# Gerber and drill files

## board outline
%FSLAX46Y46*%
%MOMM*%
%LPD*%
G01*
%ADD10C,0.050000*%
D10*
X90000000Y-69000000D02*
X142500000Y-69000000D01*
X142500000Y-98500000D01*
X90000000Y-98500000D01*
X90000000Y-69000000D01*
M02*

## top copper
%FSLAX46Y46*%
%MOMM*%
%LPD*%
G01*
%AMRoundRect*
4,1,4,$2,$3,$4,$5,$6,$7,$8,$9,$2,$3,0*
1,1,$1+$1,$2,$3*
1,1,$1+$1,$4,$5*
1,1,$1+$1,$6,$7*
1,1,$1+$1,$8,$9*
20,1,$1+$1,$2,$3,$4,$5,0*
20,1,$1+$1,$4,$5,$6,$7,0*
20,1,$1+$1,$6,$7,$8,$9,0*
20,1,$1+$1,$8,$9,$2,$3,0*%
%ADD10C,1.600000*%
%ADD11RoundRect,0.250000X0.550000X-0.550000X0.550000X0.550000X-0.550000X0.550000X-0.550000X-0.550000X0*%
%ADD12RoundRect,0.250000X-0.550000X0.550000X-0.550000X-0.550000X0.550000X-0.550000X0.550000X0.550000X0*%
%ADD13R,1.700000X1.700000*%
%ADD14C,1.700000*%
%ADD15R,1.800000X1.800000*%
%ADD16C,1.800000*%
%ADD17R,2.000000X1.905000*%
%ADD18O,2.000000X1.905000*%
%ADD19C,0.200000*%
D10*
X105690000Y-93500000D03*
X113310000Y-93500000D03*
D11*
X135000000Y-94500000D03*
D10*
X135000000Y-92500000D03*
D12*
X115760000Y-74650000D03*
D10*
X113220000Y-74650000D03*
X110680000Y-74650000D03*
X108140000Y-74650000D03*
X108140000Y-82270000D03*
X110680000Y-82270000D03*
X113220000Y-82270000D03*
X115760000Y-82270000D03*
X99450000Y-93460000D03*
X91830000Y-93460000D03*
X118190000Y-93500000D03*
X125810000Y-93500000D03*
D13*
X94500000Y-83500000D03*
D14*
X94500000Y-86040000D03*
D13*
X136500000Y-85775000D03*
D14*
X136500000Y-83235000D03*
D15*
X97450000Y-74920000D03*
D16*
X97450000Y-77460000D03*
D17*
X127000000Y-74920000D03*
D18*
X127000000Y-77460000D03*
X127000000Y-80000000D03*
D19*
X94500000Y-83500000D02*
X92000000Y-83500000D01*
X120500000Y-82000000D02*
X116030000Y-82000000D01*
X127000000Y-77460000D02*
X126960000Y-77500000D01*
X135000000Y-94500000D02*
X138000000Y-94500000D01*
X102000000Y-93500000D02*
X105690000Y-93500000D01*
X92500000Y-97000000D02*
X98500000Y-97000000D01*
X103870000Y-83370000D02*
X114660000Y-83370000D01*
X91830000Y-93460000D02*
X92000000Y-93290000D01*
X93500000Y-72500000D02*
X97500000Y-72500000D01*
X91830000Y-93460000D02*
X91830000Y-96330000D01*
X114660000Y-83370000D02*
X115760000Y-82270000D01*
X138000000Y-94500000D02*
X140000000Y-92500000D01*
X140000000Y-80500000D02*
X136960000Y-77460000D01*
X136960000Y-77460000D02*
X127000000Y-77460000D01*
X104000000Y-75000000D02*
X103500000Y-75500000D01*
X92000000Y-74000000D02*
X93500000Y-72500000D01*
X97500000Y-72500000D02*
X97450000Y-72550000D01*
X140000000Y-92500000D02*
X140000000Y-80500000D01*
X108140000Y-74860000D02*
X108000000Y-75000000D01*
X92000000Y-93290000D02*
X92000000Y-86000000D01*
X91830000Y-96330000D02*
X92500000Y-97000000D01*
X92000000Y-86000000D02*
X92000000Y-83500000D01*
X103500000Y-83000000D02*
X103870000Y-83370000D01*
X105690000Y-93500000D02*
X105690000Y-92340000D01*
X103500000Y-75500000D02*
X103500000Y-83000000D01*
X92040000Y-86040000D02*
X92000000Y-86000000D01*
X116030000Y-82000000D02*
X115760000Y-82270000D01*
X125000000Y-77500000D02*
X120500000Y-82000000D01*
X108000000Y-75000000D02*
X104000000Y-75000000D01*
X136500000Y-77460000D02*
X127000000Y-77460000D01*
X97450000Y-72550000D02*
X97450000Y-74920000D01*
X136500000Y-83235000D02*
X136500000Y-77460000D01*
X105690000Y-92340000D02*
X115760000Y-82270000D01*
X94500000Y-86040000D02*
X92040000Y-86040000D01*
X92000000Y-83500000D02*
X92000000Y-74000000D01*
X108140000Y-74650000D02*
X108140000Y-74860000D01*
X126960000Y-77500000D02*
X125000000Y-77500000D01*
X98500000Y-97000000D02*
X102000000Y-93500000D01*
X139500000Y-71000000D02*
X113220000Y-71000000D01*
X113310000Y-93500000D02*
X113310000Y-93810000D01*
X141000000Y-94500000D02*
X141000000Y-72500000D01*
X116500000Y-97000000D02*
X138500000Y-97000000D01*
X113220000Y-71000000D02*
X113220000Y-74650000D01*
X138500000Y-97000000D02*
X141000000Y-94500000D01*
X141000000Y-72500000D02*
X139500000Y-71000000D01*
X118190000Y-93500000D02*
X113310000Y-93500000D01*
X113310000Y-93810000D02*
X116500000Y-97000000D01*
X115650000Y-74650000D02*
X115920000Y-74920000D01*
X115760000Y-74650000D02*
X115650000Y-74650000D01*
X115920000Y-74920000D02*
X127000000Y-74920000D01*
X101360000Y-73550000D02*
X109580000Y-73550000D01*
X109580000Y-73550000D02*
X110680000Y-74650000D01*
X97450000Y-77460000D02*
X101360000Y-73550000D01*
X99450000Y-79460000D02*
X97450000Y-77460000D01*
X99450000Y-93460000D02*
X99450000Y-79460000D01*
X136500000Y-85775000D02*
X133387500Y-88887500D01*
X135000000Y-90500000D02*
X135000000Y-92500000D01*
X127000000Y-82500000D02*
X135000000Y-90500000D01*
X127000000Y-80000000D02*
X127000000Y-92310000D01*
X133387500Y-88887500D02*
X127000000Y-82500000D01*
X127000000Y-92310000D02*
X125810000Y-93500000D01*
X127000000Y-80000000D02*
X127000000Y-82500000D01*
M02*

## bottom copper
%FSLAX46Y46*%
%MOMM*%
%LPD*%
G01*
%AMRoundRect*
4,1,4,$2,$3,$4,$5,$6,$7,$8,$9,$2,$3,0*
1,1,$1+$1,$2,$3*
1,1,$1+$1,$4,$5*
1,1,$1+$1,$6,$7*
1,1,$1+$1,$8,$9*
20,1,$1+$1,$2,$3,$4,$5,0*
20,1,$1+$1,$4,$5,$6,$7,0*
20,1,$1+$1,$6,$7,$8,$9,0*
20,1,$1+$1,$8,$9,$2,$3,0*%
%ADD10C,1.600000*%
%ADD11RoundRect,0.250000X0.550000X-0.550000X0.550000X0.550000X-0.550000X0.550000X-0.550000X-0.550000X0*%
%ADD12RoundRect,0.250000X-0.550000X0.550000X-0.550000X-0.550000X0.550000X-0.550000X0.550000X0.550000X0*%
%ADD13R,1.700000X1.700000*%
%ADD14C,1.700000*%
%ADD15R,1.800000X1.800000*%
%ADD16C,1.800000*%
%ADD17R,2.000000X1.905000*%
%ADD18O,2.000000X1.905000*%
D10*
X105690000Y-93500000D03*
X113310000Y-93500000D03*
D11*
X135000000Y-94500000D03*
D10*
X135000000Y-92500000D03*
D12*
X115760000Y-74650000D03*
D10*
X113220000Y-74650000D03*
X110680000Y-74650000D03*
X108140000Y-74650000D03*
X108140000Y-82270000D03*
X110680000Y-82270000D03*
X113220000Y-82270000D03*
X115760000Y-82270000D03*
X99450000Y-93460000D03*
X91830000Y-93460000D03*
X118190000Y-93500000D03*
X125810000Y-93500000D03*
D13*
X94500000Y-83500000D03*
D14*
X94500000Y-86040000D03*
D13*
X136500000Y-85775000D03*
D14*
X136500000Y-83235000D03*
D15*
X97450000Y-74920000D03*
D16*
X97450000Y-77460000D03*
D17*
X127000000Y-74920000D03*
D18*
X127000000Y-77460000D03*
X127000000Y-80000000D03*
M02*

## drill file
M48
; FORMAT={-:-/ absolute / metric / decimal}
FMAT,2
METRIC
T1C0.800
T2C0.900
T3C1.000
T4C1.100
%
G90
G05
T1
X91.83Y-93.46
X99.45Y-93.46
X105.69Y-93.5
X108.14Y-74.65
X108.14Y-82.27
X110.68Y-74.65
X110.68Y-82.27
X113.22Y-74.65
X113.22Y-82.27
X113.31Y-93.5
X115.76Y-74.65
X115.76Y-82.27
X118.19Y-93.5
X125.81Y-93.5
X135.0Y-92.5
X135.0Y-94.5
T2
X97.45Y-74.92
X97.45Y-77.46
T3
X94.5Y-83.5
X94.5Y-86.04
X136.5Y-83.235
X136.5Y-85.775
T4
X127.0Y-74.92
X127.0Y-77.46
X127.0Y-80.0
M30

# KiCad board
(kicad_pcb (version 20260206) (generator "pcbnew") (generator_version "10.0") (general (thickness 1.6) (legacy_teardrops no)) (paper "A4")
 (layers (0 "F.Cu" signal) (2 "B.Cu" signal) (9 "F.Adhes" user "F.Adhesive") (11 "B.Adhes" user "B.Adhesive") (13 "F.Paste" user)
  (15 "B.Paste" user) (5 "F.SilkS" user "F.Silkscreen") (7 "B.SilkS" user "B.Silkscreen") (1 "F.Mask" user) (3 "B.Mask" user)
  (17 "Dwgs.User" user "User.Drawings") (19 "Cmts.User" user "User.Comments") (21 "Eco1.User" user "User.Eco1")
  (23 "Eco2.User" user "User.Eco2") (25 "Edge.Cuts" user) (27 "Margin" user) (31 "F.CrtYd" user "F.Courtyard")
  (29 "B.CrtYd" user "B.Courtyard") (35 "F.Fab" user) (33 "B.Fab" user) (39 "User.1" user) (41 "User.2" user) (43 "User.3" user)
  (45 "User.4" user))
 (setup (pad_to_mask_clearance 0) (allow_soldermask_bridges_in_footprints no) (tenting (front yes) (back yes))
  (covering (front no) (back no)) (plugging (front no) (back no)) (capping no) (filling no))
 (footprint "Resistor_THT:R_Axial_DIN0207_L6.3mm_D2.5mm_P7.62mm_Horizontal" (layer "F.Cu") (at 105.69 93.5)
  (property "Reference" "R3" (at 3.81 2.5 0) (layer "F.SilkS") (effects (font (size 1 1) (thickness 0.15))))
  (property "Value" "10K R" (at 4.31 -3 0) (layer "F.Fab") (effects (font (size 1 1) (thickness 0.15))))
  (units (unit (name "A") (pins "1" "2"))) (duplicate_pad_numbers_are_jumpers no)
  (pad "1" thru_hole circle (at 0 0) (size 1.6 1.6) (drill 0.8) (layers "*.Cu" "*.Mask") (remove_unused_layers no) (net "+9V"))
  (pad "2" thru_hole circle (at 7.62 0) (size 1.6 1.6) (drill 0.8) (layers "*.Cu" "*.Mask") (remove_unused_layers no) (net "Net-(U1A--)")))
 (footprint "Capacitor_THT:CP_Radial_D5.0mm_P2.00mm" (layer "F.Cu") (at 135 94.5 90)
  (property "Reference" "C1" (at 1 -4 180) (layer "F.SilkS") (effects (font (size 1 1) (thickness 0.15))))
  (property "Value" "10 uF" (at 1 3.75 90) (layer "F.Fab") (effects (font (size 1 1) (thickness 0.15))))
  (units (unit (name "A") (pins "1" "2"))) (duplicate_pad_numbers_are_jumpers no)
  (pad "1" thru_hole roundrect (at 0 0 90) (size 1.6 1.6) (drill 0.8) (layers "*.Cu" "*.Mask") (remove_unused_layers no)
   (roundrect_rratio 0.15625) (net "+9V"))
  (pad "2" thru_hole circle (at 2 0 90) (size 1.6 1.6) (drill 0.8) (layers "*.Cu" "*.Mask") (remove_unused_layers no) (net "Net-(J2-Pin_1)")))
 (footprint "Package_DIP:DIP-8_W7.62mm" (layer "F.Cu") (at 115.76 74.65 -90)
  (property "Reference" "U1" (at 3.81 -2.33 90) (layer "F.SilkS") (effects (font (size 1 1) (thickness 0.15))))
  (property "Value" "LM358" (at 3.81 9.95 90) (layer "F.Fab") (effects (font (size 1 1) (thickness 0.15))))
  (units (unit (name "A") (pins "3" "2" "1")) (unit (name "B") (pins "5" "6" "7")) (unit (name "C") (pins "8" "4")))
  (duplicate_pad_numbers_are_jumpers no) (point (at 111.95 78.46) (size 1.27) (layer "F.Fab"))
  (pad "1" thru_hole roundrect (at 0 0 270) (size 1.6 1.6) (drill 0.8) (layers "*.Cu" "*.Mask") (remove_unused_layers no)
   (roundrect_rratio 0.15625) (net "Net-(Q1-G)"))
  (pad "2" thru_hole circle (at 0 2.54 270) (size 1.6 1.6) (drill 0.8) (layers "*.Cu" "*.Mask") (remove_unused_layers no)
   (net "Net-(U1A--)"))
  (pad "3" thru_hole circle (at 0 5.08 270) (size 1.6 1.6) (drill 0.8) (layers "*.Cu" "*.Mask") (remove_unused_layers no) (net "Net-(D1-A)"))
  (pad "4" thru_hole circle (at 0 7.62 270) (size 1.6 1.6) (drill 0.8) (layers "*.Cu" "*.Mask") (remove_unused_layers no) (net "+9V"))
  (pad "5" thru_hole circle (at 7.62 7.62 270) (size 1.6 1.6) (drill 0.8) (layers "*.Cu" "*.Mask") (remove_unused_layers no))
  (pad "6" thru_hole circle (at 7.62 5.08 270) (size 1.6 1.6) (drill 0.8) (layers "*.Cu" "*.Mask") (remove_unused_layers no))
  (pad "7" thru_hole circle (at 7.62 2.54 270) (size 1.6 1.6) (drill 0.8) (layers "*.Cu" "*.Mask") (remove_unused_layers no))
  (pad "8" thru_hole circle (at 7.62 0 270) (size 1.6 1.6) (drill 0.8) (layers "*.Cu" "*.Mask") (remove_unused_layers no) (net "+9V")))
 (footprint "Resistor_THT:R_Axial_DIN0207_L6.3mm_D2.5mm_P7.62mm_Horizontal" (layer "F.Cu") (at 99.45 93.46 180)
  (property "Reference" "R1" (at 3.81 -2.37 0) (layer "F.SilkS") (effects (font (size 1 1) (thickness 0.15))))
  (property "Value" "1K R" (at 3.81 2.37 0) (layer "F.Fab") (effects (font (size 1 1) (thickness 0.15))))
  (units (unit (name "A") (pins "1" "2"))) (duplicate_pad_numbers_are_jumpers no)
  (pad "1" thru_hole circle (at 0 0 180) (size 1.6 1.6) (drill 0.8) (layers "*.Cu" "*.Mask") (remove_unused_layers no) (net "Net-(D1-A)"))
  (pad "2" thru_hole circle (at 7.62 0 180) (size 1.6 1.6) (drill 0.8) (layers "*.Cu" "*.Mask") (remove_unused_layers no) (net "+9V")))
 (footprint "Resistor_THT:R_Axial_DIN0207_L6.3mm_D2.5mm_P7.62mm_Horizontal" (layer "F.Cu") (at 118.19 93.5)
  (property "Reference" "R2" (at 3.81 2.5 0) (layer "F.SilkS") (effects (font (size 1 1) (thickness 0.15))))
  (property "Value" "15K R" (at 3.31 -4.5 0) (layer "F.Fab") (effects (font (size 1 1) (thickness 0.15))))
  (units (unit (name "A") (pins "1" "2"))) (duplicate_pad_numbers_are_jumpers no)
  (pad "1" thru_hole circle (at 0 0) (size 1.6 1.6) (drill 0.8) (layers "*.Cu" "*.Mask") (remove_unused_layers no) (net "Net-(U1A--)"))
  (pad "2" thru_hole circle (at 7.62 0) (size 1.6 1.6) (drill 0.8) (layers "*.Cu" "*.Mask") (remove_unused_layers no) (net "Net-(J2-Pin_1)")))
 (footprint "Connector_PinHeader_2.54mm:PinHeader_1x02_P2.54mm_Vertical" (layer "F.Cu") (at 94.5 83.5)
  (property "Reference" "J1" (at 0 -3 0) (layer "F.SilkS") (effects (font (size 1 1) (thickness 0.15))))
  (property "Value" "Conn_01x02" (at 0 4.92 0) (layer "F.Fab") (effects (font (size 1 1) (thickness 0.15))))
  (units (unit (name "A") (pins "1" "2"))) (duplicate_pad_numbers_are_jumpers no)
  (pad "1" thru_hole rect (at 0 0) (size 1.7 1.7) (drill 1) (layers "*.Cu" "*.Mask") (remove_unused_layers no) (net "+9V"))
  (pad "2" thru_hole circle (at 0 2.54) (size 1.7 1.7) (drill 1) (layers "*.Cu" "*.Mask") (remove_unused_layers no) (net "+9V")))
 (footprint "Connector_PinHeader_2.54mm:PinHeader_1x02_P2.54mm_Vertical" (layer "F.Cu") (at 136.5 85.775 180)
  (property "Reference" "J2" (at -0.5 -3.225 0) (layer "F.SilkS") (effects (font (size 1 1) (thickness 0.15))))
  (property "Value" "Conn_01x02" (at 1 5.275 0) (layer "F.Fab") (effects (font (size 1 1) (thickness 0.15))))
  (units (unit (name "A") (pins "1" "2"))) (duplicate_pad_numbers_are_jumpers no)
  (pad "1" thru_hole rect (at 0 0 180) (size 1.7 1.7) (drill 1) (layers "*.Cu" "*.Mask") (remove_unused_layers no) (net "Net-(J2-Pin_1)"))
  (pad "2" thru_hole circle (at 0 2.54 180) (size 1.7 1.7) (drill 1) (layers "*.Cu" "*.Mask") (remove_unused_layers no) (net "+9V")))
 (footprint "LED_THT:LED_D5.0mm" (layer "F.Cu") (at 97.45 74.92 -90)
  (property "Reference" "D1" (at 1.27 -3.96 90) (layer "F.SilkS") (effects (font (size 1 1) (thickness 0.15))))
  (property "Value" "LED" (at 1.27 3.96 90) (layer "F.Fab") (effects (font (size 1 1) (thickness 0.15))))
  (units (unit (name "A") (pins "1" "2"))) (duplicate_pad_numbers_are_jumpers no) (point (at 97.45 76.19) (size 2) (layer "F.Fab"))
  (pad "1" thru_hole rect (at 0 0 270) (size 1.8 1.8) (drill 0.9) (layers "*.Cu" "*.Mask") (remove_unused_layers no) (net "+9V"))
  (pad "2" thru_hole circle (at 2.54 0 270) (size 1.8 1.8) (drill 0.9) (layers "*.Cu" "*.Mask") (remove_unused_layers no) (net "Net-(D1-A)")))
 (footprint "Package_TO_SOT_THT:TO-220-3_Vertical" (layer "F.Cu") (at 127 74.92 -90)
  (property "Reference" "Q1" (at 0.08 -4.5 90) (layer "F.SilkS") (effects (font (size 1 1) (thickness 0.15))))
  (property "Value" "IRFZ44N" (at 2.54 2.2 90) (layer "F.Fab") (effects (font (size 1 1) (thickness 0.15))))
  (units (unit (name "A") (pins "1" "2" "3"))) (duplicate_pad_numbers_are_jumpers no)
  (pad "1" thru_hole rect (at 0 0 270) (size 1.905 2) (drill 1.1) (layers "*.Cu" "*.Mask") (remove_unused_layers no) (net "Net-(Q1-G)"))
  (pad "2" thru_hole oval (at 2.54 0 270) (size 1.905 2) (drill 1.1) (layers "*.Cu" "*.Mask") (remove_unused_layers no) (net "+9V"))
  (pad "3" thru_hole oval (at 5.08 0 270) (size 1.905 2) (drill 1.1) (layers "*.Cu" "*.Mask") (remove_unused_layers no)
   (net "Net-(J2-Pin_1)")))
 (gr_rect (start 90 69) (end 142.5 98.5) (stroke (width 0.05) (type default)) (fill no) (layer "Edge.Cuts"))
 (segment (start 94.5 83.5) (end 92 83.5) (width 0.2) (layer "F.Cu") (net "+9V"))
 (segment (start 120.5 82) (end 116.03 82) (width 0.2) (layer "F.Cu") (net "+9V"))
 (segment (start 127 77.46) (end 126.96 77.5) (width 0.2) (layer "F.Cu") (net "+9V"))
 (segment (start 135 94.5) (end 138 94.5) (width 0.2) (layer "F.Cu") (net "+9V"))
 (segment (start 102 93.5) (end 105.69 93.5) (width 0.2) (layer "F.Cu") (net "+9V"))
 (segment (start 92.5 97) (end 98.5 97) (width 0.2) (layer "F.Cu") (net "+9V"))
 (segment (start 103.87 83.37) (end 114.66 83.37) (width 0.2) (layer "F.Cu") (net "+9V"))
 (segment (start 91.83 93.46) (end 92 93.29) (width 0.2) (layer "F.Cu") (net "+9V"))
 (segment (start 93.5 72.5) (end 97.5 72.5) (width 0.2) (layer "F.Cu") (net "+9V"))
 (segment (start 91.83 93.46) (end 91.83 96.33) (width 0.2) (layer "F.Cu") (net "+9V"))
 (segment (start 114.66 83.37) (end 115.76 82.27) (width 0.2) (layer "F.Cu") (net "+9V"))
 (segment (start 138 94.5) (end 140 92.5) (width 0.2) (layer "F.Cu") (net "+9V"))
 (segment (start 140 80.5) (end 136.96 77.46) (width 0.2) (layer "F.Cu") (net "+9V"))
 (segment (start 136.96 77.46) (end 127 77.46) (width 0.2) (layer "F.Cu") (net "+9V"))
 (segment (start 104 75) (end 103.5 75.5) (width 0.2) (layer "F.Cu") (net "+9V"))
 (segment (start 92 74) (end 93.5 72.5) (width 0.2) (layer "F.Cu") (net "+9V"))
 (segment (start 97.5 72.5) (end 97.45 72.55) (width 0.2) (layer "F.Cu") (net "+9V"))
 (segment (start 140 92.5) (end 140 80.5) (width 0.2) (layer "F.Cu") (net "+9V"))
 (segment (start 108.14 74.86) (end 108 75) (width 0.2) (layer "F.Cu") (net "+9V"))
 (segment (start 92 93.29) (end 92 86) (width 0.2) (layer "F.Cu") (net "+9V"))
 (segment (start 91.83 96.33) (end 92.5 97) (width 0.2) (layer "F.Cu") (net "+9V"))
 (segment (start 92 86) (end 92 83.5) (width 0.2) (layer "F.Cu") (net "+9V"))
 (segment (start 103.5 83) (end 103.87 83.37) (width 0.2) (layer "F.Cu") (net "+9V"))
 (segment (start 105.69 93.5) (end 105.69 92.34) (width 0.2) (layer "F.Cu") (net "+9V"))
 (segment (start 103.5 75.5) (end 103.5 83) (width 0.2) (layer "F.Cu") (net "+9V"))
 (segment (start 92.04 86.04) (end 92 86) (width 0.2) (layer "F.Cu") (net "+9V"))
 (segment (start 116.03 82) (end 115.76 82.27) (width 0.2) (layer "F.Cu") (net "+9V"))
 (segment (start 125 77.5) (end 120.5 82) (width 0.2) (layer "F.Cu") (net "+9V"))
 (segment (start 108 75) (end 104 75) (width 0.2) (layer "F.Cu") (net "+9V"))
 (segment (start 136.5 77.46) (end 127 77.46) (width 0.2) (layer "F.Cu") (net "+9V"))
 (segment (start 97.45 72.55) (end 97.45 74.92) (width 0.2) (layer "F.Cu") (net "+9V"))
 (segment (start 136.5 83.235) (end 136.5 77.46) (width 0.2) (layer "F.Cu") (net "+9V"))
 (segment (start 105.69 92.34) (end 115.76 82.27) (width 0.2) (layer "F.Cu") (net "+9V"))
 (segment (start 94.5 86.04) (end 92.04 86.04) (width 0.2) (layer "F.Cu") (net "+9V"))
 (segment (start 92 83.5) (end 92 74) (width 0.2) (layer "F.Cu") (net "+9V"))
 (segment (start 108.14 74.65) (end 108.14 74.86) (width 0.2) (layer "F.Cu") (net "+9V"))
 (segment (start 126.96 77.5) (end 125 77.5) (width 0.2) (layer "F.Cu") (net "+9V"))
 (segment (start 98.5 97) (end 102 93.5) (width 0.2) (layer "F.Cu") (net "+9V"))
 (segment (start 139.5 71) (end 113.22 71) (width 0.2) (layer "F.Cu") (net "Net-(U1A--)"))
 (segment (start 113.31 93.5) (end 113.31 93.81) (width 0.2) (layer "F.Cu") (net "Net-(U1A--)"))
 (segment (start 141 94.5) (end 141 72.5) (width 0.2) (layer "F.Cu") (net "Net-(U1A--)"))
 (segment (start 116.5 97) (end 138.5 97) (width 0.2) (layer "F.Cu") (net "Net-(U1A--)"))
 (segment (start 113.22 71) (end 113.22 74.65) (width 0.2) (layer "F.Cu") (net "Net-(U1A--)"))
 (segment (start 138.5 97) (end 141 94.5) (width 0.2) (layer "F.Cu") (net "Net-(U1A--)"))
 (segment (start 141 72.5) (end 139.5 71) (width 0.2) (layer "F.Cu") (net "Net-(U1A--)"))
 (segment (start 118.19 93.5) (end 113.31 93.5) (width 0.2) (layer "F.Cu") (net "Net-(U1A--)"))
 (segment (start 113.31 93.81) (end 116.5 97) (width 0.2) (layer "F.Cu") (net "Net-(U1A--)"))
 (segment (start 115.65 74.65) (end 115.92 74.92) (width 0.2) (layer "F.Cu") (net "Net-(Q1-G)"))
 (segment (start 115.76 74.65) (end 115.65 74.65) (width 0.2) (layer "F.Cu") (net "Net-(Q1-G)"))
 (segment (start 115.92 74.92) (end 127 74.92) (width 0.2) (layer "F.Cu") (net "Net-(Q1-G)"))
 (segment (start 101.36 73.55) (end 109.58 73.55) (width 0.2) (layer "F.Cu") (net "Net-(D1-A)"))
 (segment (start 109.58 73.55) (end 110.68 74.65) (width 0.2) (layer "F.Cu") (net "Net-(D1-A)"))
 (segment (start 97.45 77.46) (end 101.36 73.55) (width 0.2) (layer "F.Cu") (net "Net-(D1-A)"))
 (segment (start 99.45 79.46) (end 97.45 77.46) (width 0.2) (layer "F.Cu") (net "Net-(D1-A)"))
 (segment (start 99.45 93.46) (end 99.45 79.46) (width 0.2) (layer "F.Cu") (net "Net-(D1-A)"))
 (segment (start 136.5 85.775) (end 133.3875 88.8875) (width 0.2) (layer "F.Cu") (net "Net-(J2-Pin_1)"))
 (segment (start 135 90.5) (end 135 92.5) (width 0.2) (layer "F.Cu") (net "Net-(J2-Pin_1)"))
 (segment (start 127 82.5) (end 135 90.5) (width 0.2) (layer "F.Cu") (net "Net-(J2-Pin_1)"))
 (segment (start 127 80) (end 127 92.31) (width 0.2) (layer "F.Cu") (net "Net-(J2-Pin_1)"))
 (segment (start 133.3875 88.8875) (end 127 82.5) (width 0.2) (layer "F.Cu") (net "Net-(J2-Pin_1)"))
 (segment (start 127 92.31) (end 125.81 93.5) (width 0.2) (layer "F.Cu") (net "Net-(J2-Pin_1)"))
 (segment (start 127 80) (end 127 82.5) (width 0.2) (layer "F.Cu") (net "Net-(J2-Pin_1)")))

